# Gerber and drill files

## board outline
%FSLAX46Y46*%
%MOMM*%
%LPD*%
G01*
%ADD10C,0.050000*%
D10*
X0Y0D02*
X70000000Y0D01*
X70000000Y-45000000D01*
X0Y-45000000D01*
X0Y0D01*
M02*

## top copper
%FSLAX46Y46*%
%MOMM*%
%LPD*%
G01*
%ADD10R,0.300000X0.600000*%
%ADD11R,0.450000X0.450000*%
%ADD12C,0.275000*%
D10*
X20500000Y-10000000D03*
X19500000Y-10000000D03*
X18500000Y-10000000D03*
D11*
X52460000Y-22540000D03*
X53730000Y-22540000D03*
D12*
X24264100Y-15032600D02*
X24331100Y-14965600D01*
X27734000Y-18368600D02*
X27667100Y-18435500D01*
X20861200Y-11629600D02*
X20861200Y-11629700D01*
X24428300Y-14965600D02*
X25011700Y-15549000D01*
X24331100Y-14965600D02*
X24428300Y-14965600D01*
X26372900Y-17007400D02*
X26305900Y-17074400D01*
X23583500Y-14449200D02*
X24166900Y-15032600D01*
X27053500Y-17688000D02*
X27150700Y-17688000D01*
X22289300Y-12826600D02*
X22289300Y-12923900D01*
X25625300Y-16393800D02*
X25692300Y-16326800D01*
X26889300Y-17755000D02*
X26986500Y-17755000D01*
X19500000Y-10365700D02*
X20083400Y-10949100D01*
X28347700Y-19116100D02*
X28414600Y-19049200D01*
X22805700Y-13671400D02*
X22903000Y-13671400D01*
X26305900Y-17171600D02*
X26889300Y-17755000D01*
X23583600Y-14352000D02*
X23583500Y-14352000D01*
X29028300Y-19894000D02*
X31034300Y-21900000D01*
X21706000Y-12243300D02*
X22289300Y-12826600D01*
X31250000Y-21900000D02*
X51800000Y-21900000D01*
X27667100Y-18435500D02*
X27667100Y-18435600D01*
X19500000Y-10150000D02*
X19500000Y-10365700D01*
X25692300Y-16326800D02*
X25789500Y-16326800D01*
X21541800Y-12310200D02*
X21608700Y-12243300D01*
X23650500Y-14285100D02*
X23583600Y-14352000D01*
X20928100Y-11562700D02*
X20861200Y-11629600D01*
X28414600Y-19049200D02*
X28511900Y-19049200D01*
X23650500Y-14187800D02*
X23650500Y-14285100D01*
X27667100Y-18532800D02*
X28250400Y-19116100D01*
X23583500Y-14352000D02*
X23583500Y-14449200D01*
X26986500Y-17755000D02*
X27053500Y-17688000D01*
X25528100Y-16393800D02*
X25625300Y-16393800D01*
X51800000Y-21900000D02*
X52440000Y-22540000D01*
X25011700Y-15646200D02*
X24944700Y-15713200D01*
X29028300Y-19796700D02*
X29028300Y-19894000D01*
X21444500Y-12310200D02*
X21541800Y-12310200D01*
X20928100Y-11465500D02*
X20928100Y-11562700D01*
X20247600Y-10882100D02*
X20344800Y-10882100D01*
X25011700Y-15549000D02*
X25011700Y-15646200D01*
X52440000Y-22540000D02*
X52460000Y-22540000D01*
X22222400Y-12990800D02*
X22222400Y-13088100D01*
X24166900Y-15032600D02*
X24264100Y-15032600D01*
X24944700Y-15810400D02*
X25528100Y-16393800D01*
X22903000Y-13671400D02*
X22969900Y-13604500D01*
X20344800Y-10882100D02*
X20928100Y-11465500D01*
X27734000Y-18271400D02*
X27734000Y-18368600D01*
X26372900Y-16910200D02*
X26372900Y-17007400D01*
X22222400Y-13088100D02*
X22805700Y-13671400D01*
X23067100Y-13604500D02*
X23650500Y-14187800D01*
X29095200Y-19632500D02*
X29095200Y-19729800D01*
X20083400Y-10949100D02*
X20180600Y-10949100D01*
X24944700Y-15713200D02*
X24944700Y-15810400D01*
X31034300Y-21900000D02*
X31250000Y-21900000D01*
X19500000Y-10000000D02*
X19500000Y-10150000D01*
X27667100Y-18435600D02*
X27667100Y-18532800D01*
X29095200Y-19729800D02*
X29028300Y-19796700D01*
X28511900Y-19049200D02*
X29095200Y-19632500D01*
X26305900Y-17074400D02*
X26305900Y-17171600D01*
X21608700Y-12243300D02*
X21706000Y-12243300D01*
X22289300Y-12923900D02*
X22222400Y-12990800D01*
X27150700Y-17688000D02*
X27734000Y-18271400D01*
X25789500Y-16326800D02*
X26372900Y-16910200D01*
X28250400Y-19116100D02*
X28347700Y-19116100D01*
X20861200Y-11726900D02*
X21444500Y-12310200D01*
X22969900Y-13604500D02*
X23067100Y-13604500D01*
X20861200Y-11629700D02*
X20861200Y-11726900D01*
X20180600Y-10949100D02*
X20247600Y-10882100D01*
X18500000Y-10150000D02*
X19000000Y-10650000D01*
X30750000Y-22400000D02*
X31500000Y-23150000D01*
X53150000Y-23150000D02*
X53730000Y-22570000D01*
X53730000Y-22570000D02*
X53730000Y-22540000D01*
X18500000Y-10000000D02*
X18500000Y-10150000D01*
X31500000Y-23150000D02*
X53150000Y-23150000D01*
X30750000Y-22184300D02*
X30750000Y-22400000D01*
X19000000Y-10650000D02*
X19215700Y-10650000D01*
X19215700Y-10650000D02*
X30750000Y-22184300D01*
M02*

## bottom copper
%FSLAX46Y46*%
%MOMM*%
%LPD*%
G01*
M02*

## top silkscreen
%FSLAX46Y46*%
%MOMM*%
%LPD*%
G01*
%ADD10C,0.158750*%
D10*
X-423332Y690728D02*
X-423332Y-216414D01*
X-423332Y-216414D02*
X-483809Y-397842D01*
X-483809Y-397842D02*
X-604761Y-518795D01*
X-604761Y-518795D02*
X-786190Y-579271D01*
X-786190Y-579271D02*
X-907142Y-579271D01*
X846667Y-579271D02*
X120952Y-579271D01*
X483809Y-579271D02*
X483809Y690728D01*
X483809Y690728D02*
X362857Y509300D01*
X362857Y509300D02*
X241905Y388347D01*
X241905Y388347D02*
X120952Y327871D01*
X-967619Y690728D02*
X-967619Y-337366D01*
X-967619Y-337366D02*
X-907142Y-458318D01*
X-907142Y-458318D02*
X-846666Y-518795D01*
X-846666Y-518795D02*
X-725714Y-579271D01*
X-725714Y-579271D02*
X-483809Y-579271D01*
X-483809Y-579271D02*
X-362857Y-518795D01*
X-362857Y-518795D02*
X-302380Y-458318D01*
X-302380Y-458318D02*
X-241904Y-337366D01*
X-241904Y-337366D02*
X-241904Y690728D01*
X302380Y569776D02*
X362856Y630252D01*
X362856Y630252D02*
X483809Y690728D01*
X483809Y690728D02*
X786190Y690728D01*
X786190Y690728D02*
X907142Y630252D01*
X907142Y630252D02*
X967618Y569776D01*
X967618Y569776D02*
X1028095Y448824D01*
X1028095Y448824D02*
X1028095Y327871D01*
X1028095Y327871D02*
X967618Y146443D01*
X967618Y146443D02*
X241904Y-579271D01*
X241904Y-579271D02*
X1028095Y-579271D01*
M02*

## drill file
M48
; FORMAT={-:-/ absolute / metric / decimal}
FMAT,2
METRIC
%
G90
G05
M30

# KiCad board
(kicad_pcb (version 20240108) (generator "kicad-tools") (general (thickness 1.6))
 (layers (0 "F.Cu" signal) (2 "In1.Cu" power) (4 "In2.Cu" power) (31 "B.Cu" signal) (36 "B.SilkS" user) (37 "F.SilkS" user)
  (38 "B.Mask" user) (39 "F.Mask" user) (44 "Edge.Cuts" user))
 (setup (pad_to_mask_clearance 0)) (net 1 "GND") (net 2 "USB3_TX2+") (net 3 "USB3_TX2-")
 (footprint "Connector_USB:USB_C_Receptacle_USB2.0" (layer "F.Cu") (at 0 0) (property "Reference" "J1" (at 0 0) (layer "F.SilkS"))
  (pad "B1" smd rect (at 20.5 10) (size 0.3 0.6) (layers "F.Cu" "F.Mask") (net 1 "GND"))
  (pad "B2" smd rect (at 19.5 10) (size 0.3 0.6) (layers "F.Cu" "F.Mask") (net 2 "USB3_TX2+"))
  (pad "B3" smd rect (at 18.5 10) (size 0.3 0.6) (layers "F.Cu" "F.Mask") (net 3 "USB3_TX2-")))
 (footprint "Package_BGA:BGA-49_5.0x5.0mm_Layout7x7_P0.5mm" (layer "F.Cu") (at 0 0) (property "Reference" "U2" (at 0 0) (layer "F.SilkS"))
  (pad "F2" smd rect (at 52.46 22.54) (size 0.45 0.45) (layers "F.Cu" "F.Mask") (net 2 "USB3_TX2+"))
  (pad "F3" smd rect (at 53.73 22.54) (size 0.45 0.45) (layers "F.Cu" "F.Mask") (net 3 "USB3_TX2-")))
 (segment (start 24.2641 15.0326) (end 24.3311 14.9656) (width 0.275) (layer "F.Cu") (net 2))
 (segment (start 27.734 18.3686) (end 27.6671 18.4355) (width 0.275) (layer "F.Cu") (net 2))
 (segment (start 20.8612 11.6296) (end 20.8612 11.6297) (width 0.275) (layer "F.Cu") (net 2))
 (segment (start 24.4283 14.9656) (end 25.0117 15.549) (width 0.275) (layer "F.Cu") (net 2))
 (segment (start 24.3311 14.9656) (end 24.4283 14.9656) (width 0.275) (layer "F.Cu") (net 2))
 (segment (start 26.3729 17.0074) (end 26.3059 17.0744) (width 0.275) (layer "F.Cu") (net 2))
 (segment (start 23.5835 14.4492) (end 24.1669 15.0326) (width 0.275) (layer "F.Cu") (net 2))
 (segment (start 27.0535 17.688) (end 27.1507 17.688) (width 0.275) (layer "F.Cu") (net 2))
 (segment (start 22.2893 12.8266) (end 22.2893 12.9239) (width 0.275) (layer "F.Cu") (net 2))
 (segment (start 25.6253 16.3938) (end 25.6923 16.3268) (width 0.275) (layer "F.Cu") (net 2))
 (segment (start 26.8893 17.755) (end 26.9865 17.755) (width 0.275) (layer "F.Cu") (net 2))
 (segment (start 19.5 10.3657) (end 20.0834 10.9491) (width 0.275) (layer "F.Cu") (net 2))
 (segment (start 28.3477 19.1161) (end 28.4146 19.0492) (width 0.275) (layer "F.Cu") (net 2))
 (segment (start 22.8057 13.6714) (end 22.903 13.6714) (width 0.275) (layer "F.Cu") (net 2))
 (segment (start 26.3059 17.1716) (end 26.8893 17.755) (width 0.275) (layer "F.Cu") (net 2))
 (segment (start 23.5836 14.352) (end 23.5835 14.352) (width 0.275) (layer "F.Cu") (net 2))
 (segment (start 29.0283 19.894) (end 31.0343 21.9) (width 0.275) (layer "F.Cu") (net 2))
 (segment (start 21.706 12.2433) (end 22.2893 12.8266) (width 0.275) (layer "F.Cu") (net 2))
 (segment (start 31.25 21.9) (end 51.8 21.9) (width 0.275) (layer "F.Cu") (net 2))
 (segment (start 27.6671 18.4355) (end 27.6671 18.4356) (width 0.275) (layer "F.Cu") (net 2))
 (segment (start 19.5 10.15) (end 19.5 10.3657) (width 0.275) (layer "F.Cu") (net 2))
 (segment (start 25.6923 16.3268) (end 25.7895 16.3268) (width 0.275) (layer "F.Cu") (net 2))
 (segment (start 21.5418 12.3102) (end 21.6087 12.2433) (width 0.275) (layer "F.Cu") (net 2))
 (segment (start 23.6505 14.2851) (end 23.5836 14.352) (width 0.275) (layer "F.Cu") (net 2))
 (segment (start 20.9281 11.5627) (end 20.8612 11.6296) (width 0.275) (layer "F.Cu") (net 2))
 (segment (start 28.4146 19.0492) (end 28.5119 19.0492) (width 0.275) (layer "F.Cu") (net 2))
 (segment (start 23.6505 14.1878) (end 23.6505 14.2851) (width 0.275) (layer "F.Cu") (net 2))
 (segment (start 27.6671 18.5328) (end 28.2504 19.1161) (width 0.275) (layer "F.Cu") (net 2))
 (segment (start 23.5835 14.352) (end 23.5835 14.4492) (width 0.275) (layer "F.Cu") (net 2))
 (segment (start 26.9865 17.755) (end 27.0535 17.688) (width 0.275) (layer "F.Cu") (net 2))
 (segment (start 25.5281 16.3938) (end 25.6253 16.3938) (width 0.275) (layer "F.Cu") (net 2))
 (segment (start 51.8 21.9) (end 52.44 22.54) (width 0.275) (layer "F.Cu") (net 2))
 (segment (start 25.0117 15.6462) (end 24.9447 15.7132) (width 0.275) (layer "F.Cu") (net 2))
 (segment (start 29.0283 19.7967) (end 29.0283 19.894) (width 0.275) (layer "F.Cu") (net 2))
 (segment (start 21.4445 12.3102) (end 21.5418 12.3102) (width 0.275) (layer "F.Cu") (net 2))
 (segment (start 20.9281 11.4655) (end 20.9281 11.5627) (width 0.275) (layer "F.Cu") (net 2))
 (segment (start 20.2476 10.8821) (end 20.3448 10.8821) (width 0.275) (layer "F.Cu") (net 2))
 (segment (start 25.0117 15.549) (end 25.0117 15.6462) (width 0.275) (layer "F.Cu") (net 2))
 (segment (start 52.44 22.54) (end 52.46 22.54) (width 0.275) (layer "F.Cu") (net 2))
 (segment (start 22.2224 12.9908) (end 22.2224 13.0881) (width 0.275) (layer "F.Cu") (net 2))
 (segment (start 24.1669 15.0326) (end 24.2641 15.0326) (width 0.275) (layer "F.Cu") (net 2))
 (segment (start 24.9447 15.8104) (end 25.5281 16.3938) (width 0.275) (layer "F.Cu") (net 2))
 (segment (start 22.903 13.6714) (end 22.9699 13.6045) (width 0.275) (layer "F.Cu") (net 2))
 (segment (start 20.3448 10.8821) (end 20.9281 11.4655) (width 0.275) (layer "F.Cu") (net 2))
 (segment (start 27.734 18.2714) (end 27.734 18.3686) (width 0.275) (layer "F.Cu") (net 2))
 (segment (start 26.3729 16.9102) (end 26.3729 17.0074) (width 0.275) (layer "F.Cu") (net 2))
 (segment (start 22.2224 13.0881) (end 22.8057 13.6714) (width 0.275) (layer "F.Cu") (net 2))
 (segment (start 23.0671 13.6045) (end 23.6505 14.1878) (width 0.275) (layer "F.Cu") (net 2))
 (segment (start 29.0952 19.6325) (end 29.0952 19.7298) (width 0.275) (layer "F.Cu") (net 2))
 (segment (start 20.0834 10.9491) (end 20.1806 10.9491) (width 0.275) (layer "F.Cu") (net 2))
 (segment (start 24.9447 15.7132) (end 24.9447 15.8104) (width 0.275) (layer "F.Cu") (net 2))
 (segment (start 31.0343 21.9) (end 31.25 21.9) (width 0.275) (layer "F.Cu") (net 2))
 (segment (start 19.5 10) (end 19.5 10.15) (width 0.275) (layer "F.Cu") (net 2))
 (segment (start 27.6671 18.4356) (end 27.6671 18.5328) (width 0.275) (layer "F.Cu") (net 2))
 (segment (start 29.0952 19.7298) (end 29.0283 19.7967) (width 0.275) (layer "F.Cu") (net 2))
 (segment (start 28.5119 19.0492) (end 29.0952 19.6325) (width 0.275) (layer "F.Cu") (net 2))
 (segment (start 26.3059 17.0744) (end 26.3059 17.1716) (width 0.275) (layer "F.Cu") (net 2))
 (segment (start 21.6087 12.2433) (end 21.706 12.2433) (width 0.275) (layer "F.Cu") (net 2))
 (segment (start 22.2893 12.9239) (end 22.2224 12.9908) (width 0.275) (layer "F.Cu") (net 2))
 (segment (start 27.1507 17.688) (end 27.734 18.2714) (width 0.275) (layer "F.Cu") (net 2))
 (segment (start 25.7895 16.3268) (end 26.3729 16.9102) (width 0.275) (layer "F.Cu") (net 2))
 (segment (start 28.2504 19.1161) (end 28.3477 19.1161) (width 0.275) (layer "F.Cu") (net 2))
 (segment (start 20.8612 11.7269) (end 21.4445 12.3102) (width 0.275) (layer "F.Cu") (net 2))
 (segment (start 22.9699 13.6045) (end 23.0671 13.6045) (width 0.275) (layer "F.Cu") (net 2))
 (segment (start 20.8612 11.6297) (end 20.8612 11.7269) (width 0.275) (layer "F.Cu") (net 2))
 (segment (start 20.1806 10.9491) (end 20.2476 10.8821) (width 0.275) (layer "F.Cu") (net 2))
 (segment (start 18.5 10.15) (end 19 10.65) (width 0.275) (layer "F.Cu") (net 3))
 (segment (start 30.75 22.4) (end 31.5 23.15) (width 0.275) (layer "F.Cu") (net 3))
 (segment (start 53.15 23.15) (end 53.73 22.57) (width 0.275) (layer "F.Cu") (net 3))
 (segment (start 53.73 22.57) (end 53.73 22.54) (width 0.275) (layer "F.Cu") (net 3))
 (segment (start 18.5 10) (end 18.5 10.15) (width 0.275) (layer "F.Cu") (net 3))
 (segment (start 31.5 23.15) (end 53.15 23.15) (width 0.275) (layer "F.Cu") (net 3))
 (segment (start 30.75 22.1843) (end 30.75 22.4) (width 0.275) (layer "F.Cu") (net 3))
 (segment (start 19 10.65) (end 19.2157 10.65) (width 0.275) (layer "F.Cu") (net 3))
 (segment (start 19.2157 10.65) (end 30.75 22.1843) (width 0.275) (layer "F.Cu") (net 3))
 (gr_rect (start 0 0) (end 70 45) (stroke (width 0.05) (type default)) (fill none) (layer "Edge.Cuts")))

